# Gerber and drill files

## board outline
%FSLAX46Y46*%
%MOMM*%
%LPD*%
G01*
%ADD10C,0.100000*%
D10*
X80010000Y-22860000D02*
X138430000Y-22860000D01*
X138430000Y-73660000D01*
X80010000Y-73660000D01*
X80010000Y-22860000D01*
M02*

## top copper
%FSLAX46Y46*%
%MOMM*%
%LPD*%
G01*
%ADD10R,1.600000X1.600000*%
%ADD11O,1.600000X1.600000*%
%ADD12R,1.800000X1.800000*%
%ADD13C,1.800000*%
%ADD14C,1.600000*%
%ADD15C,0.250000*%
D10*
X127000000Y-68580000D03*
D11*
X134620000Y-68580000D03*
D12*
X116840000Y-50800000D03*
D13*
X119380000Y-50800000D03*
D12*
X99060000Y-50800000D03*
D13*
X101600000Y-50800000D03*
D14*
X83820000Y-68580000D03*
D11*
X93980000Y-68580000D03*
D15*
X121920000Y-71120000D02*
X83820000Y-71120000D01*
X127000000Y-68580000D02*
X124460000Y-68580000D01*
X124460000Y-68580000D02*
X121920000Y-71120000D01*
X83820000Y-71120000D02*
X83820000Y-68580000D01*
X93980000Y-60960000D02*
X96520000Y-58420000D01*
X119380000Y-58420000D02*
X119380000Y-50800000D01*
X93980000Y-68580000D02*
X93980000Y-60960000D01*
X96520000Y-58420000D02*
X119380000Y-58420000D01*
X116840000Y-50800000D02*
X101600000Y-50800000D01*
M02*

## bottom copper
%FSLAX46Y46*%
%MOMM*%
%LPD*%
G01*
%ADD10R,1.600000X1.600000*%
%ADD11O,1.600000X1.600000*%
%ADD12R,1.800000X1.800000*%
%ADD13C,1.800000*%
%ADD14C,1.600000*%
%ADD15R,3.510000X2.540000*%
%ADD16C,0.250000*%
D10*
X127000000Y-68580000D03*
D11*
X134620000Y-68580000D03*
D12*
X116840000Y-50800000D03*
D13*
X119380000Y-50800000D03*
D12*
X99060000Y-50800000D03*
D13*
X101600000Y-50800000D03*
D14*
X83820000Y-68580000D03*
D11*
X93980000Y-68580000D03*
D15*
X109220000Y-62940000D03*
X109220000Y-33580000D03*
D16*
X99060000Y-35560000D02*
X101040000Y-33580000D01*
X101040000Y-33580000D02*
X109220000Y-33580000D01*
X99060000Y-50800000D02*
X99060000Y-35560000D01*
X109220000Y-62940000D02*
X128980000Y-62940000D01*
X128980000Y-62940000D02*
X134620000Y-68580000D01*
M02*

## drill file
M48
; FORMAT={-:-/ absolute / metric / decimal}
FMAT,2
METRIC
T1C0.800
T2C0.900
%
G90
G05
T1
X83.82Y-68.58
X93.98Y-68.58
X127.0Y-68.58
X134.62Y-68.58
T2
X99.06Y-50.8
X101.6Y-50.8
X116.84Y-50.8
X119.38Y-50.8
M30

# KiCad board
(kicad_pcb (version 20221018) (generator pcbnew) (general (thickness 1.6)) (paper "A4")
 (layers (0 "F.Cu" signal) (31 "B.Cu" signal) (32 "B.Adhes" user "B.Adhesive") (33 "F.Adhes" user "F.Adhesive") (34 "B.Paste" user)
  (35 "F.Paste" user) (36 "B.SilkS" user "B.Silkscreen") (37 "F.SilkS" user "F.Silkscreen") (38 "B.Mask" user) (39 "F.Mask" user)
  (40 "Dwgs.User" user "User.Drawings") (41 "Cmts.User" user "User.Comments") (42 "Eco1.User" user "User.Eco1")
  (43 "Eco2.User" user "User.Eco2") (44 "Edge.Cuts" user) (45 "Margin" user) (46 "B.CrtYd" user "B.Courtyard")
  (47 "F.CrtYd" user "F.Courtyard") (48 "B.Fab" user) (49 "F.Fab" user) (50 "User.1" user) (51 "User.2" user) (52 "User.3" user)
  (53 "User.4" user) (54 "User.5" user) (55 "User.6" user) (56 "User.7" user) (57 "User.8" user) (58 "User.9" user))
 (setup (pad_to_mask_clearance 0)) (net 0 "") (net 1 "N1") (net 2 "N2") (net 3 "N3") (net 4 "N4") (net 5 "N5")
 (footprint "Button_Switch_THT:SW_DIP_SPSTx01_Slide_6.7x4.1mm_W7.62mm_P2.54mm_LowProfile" (layer "F.Cu") (at 127 68.58)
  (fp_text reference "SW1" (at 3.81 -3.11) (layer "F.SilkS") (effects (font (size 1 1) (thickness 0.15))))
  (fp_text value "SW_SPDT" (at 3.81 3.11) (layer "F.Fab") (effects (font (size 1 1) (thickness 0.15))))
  (pad "1" thru_hole rect (at 0 0) (size 1.6 1.6) (drill 0.8) (layers "*.Cu" "*.Mask") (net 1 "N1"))
  (pad "2" thru_hole oval (at 7.62 0) (size 1.6 1.6) (drill 0.8) (layers "*.Cu" "*.Mask") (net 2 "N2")))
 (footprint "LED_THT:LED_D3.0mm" (layer "F.Cu") (at 116.84 50.8)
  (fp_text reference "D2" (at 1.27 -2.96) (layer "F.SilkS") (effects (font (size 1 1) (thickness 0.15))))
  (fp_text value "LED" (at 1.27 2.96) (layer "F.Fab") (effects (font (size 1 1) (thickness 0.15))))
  (pad "1" thru_hole rect (at 0 0) (size 1.8 1.8) (drill 0.9) (layers "*.Cu" "*.Mask") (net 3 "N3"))
  (pad "2" thru_hole circle (at 2.54 0) (size 1.8 1.8) (drill 0.9) (layers "*.Cu" "*.Mask") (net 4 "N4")))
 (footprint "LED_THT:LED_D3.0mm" (layer "F.Cu") (at 99.06 50.8)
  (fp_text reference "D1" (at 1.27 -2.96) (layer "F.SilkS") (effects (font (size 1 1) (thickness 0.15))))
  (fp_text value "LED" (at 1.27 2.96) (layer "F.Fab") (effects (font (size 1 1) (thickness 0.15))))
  (pad "1" thru_hole rect (at 0 0) (size 1.8 1.8) (drill 0.9) (layers "*.Cu" "*.Mask") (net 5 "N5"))
  (pad "2" thru_hole circle (at 2.54 0) (size 1.8 1.8) (drill 0.9) (layers "*.Cu" "*.Mask") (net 3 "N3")))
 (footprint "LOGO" (layer "F.Cu") (at 109.22 48.26)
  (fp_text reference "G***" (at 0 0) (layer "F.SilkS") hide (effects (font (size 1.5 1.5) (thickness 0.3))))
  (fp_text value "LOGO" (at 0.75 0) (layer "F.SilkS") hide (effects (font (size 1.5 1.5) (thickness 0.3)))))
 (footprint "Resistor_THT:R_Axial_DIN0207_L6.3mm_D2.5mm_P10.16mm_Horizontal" (layer "F.Cu") (at 83.82 68.58)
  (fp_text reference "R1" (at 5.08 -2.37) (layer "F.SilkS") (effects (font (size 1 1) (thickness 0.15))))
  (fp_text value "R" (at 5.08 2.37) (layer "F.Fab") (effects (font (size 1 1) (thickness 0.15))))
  (pad "1" thru_hole circle (at 0 0) (size 1.6 1.6) (drill 0.8) (layers "*.Cu" "*.Mask") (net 1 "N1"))
  (pad "2" thru_hole oval (at 10.16 0) (size 1.6 1.6) (drill 0.8) (layers "*.Cu" "*.Mask") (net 4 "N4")))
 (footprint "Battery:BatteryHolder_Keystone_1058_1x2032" (layer "B.Cu") (at 109.22 48.26 90)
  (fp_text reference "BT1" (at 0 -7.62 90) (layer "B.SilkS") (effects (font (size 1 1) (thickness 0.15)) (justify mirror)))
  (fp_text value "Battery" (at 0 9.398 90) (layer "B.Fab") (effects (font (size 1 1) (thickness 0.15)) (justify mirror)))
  (pad "1" smd rect (at -14.68 0 90) (size 2.54 3.51) (layers "B.Cu" "B.Paste" "B.Mask") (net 2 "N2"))
  (pad "2" smd rect (at 14.68 0 90) (size 2.54 3.51) (layers "B.Cu" "B.Paste" "B.Mask") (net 5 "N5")))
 (gr_rect (start 80.01 22.86) (end 138.43 73.66) (stroke (width 0.1) (type default)) (fill none) (layer "Edge.Cuts"))
 (segment (start 121.92 71.12) (end 83.82 71.12) (width 0.25) (layer "F.Cu") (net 1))
 (segment (start 127 68.58) (end 124.46 68.58) (width 0.25) (layer "F.Cu") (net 1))
 (segment (start 124.46 68.58) (end 121.92 71.12) (width 0.25) (layer "F.Cu") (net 1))
 (segment (start 83.82 71.12) (end 83.82 68.58) (width 0.25) (layer "F.Cu") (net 1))
 (segment (start 93.98 60.96) (end 96.52 58.42) (width 0.25) (layer "F.Cu") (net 4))
 (segment (start 119.38 58.42) (end 119.38 50.8) (width 0.25) (layer "F.Cu") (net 4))
 (segment (start 93.98 68.58) (end 93.98 60.96) (width 0.25) (layer "F.Cu") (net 4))
 (segment (start 96.52 58.42) (end 119.38 58.42) (width 0.25) (layer "F.Cu") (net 4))
 (segment (start 99.06 35.56) (end 101.04 33.58) (width 0.25) (layer "B.Cu") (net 5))
 (segment (start 101.04 33.58) (end 109.22 33.58) (width 0.25) (layer "B.Cu") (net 5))
 (segment (start 99.06 50.8) (end 99.06 35.56) (width 0.25) (layer "B.Cu") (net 5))
 (segment (start 116.84 50.8) (end 101.6 50.8) (width 0.25) (layer "F.Cu") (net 3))
 (segment (start 109.22 62.94) (end 128.98 62.94) (width 0.25) (layer "B.Cu") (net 2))
 (segment (start 128.98 62.94) (end 134.62 68.58) (width 0.25) (layer "B.Cu") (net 2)))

